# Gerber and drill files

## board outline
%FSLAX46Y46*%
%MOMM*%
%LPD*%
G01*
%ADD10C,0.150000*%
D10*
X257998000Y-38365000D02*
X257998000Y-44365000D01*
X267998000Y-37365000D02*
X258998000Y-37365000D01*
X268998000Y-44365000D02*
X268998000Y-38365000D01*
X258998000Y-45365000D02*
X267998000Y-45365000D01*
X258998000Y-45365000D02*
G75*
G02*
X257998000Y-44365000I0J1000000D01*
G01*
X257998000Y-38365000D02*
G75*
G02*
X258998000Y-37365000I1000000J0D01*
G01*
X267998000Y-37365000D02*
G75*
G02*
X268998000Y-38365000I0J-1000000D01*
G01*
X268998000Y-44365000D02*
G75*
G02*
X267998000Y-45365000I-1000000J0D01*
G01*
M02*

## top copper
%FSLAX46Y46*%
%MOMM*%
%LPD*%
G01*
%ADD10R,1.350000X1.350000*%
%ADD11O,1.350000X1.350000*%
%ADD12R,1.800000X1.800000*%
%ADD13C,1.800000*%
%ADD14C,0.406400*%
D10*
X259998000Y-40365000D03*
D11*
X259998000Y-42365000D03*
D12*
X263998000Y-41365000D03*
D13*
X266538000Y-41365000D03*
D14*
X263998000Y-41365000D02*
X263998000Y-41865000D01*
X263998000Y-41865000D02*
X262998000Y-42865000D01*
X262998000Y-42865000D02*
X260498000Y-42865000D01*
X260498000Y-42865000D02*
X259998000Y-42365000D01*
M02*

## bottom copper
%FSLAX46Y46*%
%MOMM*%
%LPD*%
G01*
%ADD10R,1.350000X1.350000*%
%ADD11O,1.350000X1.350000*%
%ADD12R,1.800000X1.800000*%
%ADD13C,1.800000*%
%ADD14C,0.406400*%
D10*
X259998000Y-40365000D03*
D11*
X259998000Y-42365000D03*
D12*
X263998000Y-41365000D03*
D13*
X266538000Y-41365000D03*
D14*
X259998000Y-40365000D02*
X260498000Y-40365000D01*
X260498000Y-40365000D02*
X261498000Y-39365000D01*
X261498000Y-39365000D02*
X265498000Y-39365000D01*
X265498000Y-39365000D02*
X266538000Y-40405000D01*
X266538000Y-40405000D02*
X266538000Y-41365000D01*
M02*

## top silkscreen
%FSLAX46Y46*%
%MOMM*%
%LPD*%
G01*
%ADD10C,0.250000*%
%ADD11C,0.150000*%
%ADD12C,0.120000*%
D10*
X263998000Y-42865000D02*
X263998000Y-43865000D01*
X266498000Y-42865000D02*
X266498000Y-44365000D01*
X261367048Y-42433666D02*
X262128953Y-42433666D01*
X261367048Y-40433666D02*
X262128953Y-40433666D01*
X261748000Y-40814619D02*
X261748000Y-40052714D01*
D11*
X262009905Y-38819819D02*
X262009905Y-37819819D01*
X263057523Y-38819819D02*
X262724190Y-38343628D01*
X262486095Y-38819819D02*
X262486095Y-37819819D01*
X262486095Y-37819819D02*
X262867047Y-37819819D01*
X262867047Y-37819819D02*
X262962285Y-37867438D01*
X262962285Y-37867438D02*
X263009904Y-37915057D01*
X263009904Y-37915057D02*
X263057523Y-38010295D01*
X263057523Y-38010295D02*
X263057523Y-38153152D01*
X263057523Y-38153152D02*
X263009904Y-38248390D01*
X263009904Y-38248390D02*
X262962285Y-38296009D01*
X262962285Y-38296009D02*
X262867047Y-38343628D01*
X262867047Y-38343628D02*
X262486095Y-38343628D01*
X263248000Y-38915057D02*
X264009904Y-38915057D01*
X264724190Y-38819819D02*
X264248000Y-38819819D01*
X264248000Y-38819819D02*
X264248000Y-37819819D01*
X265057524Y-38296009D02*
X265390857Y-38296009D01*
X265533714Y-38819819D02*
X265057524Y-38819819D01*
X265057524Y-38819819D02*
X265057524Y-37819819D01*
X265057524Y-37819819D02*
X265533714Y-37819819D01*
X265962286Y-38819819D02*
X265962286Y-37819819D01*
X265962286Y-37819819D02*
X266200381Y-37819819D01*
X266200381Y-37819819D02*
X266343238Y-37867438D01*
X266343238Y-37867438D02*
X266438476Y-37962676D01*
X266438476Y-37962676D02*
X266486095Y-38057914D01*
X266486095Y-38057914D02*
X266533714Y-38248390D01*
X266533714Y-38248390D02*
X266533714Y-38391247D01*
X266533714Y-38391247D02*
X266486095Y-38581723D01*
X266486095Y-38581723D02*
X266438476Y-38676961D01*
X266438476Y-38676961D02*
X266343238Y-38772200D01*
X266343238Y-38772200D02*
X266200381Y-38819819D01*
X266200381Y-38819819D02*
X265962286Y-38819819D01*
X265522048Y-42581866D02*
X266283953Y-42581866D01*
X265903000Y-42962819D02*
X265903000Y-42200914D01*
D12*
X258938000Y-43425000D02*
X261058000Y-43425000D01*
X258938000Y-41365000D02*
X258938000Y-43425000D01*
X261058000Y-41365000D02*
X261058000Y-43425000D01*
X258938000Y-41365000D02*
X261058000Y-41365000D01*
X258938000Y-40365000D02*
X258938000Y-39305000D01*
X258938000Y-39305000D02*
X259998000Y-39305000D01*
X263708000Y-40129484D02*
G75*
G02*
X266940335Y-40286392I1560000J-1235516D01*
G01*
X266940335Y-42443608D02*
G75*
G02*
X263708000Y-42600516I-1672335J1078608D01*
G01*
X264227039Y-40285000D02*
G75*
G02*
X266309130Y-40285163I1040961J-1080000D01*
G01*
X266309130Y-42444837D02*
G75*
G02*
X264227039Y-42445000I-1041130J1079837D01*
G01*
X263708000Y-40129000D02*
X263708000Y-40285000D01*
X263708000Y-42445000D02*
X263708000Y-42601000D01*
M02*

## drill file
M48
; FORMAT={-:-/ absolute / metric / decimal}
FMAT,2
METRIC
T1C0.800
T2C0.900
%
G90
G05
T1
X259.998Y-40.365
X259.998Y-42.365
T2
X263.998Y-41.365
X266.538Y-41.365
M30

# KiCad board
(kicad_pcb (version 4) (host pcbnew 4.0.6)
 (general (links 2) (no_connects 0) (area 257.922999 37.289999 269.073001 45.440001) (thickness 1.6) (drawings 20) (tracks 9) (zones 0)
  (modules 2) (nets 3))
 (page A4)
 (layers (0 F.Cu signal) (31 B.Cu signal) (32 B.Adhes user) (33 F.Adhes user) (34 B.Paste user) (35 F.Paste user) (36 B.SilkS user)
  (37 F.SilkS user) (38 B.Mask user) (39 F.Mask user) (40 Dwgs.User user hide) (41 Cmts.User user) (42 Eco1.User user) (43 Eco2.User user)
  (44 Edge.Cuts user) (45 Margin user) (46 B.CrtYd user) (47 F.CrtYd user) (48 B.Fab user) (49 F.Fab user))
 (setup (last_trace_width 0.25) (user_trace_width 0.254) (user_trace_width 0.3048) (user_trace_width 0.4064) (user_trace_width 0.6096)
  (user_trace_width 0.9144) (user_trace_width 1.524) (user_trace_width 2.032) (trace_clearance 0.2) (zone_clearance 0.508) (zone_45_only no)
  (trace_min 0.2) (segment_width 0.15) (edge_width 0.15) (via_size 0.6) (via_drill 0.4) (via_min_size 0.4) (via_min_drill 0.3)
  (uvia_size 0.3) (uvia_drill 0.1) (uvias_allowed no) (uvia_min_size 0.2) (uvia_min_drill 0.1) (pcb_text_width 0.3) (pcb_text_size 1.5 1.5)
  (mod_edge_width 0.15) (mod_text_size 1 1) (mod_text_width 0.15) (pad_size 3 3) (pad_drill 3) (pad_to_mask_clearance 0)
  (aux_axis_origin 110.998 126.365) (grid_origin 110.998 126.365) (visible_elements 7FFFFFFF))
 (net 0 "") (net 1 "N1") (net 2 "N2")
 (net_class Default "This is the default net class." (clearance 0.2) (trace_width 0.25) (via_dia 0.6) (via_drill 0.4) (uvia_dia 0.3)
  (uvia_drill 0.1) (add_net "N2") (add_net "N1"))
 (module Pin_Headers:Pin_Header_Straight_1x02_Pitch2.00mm (layer F.Cu) (at 259.998 40.365)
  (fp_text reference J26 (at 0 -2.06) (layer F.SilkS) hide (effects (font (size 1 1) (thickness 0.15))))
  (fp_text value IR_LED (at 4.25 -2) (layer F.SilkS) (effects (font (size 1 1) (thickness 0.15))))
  (fp_line (start -1.06 3.06) (end 1.06 3.06) (layer F.SilkS) (width 0.12))
  (fp_line (start -1.06 1) (end -1.06 3.06) (layer F.SilkS) (width 0.12))
  (fp_line (start 1.06 1) (end 1.06 3.06) (layer F.SilkS) (width 0.12))
  (fp_line (start -1.06 1) (end 1.06 1) (layer F.SilkS) (width 0.12))
  (fp_line (start -1.06 0) (end -1.06 -1.06) (layer F.SilkS) (width 0.12))
  (fp_line (start -1.06 -1.06) (end 0 -1.06) (layer F.SilkS) (width 0.12))
  (pad 1 thru_hole rect (at 0 0) (size 1.35 1.35) (drill 0.8) (layers *.Cu *.Mask) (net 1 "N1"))
  (pad 2 thru_hole oval (at 0 2) (size 1.35 1.35) (drill 0.8) (layers *.Cu *.Mask) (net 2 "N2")))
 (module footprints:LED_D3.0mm (layer F.Cu) (at 263.998 41.365)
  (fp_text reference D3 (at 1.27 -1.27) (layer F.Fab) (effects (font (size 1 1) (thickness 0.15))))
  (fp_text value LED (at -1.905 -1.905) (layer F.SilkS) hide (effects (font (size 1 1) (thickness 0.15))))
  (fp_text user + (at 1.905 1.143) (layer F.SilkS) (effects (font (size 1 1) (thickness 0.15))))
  (fp_arc (start 1.27 0) (end -0.29 -1.235516) (angle 108.8) (layer F.SilkS) (width 0.12))
  (fp_arc (start 1.27 0) (end -0.29 1.235516) (angle -108.8) (layer F.SilkS) (width 0.12))
  (fp_arc (start 1.27 0) (end 0.229039 -1.08) (angle 87.9) (layer F.SilkS) (width 0.12))
  (fp_arc (start 1.27 0) (end 0.229039 1.08) (angle -87.9) (layer F.SilkS) (width 0.12))
  (fp_line (start -0.29 -1.236) (end -0.29 -1.08) (layer F.SilkS) (width 0.12))
  (fp_line (start -0.29 1.08) (end -0.29 1.236) (layer F.SilkS) (width 0.12))
  (pad 1 thru_hole rect (at 0 0) (size 1.8 1.8) (drill 0.9) (layers *.Cu *.Mask) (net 2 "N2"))
  (pad 2 thru_hole circle (at 2.54 0) (size 1.8 1.8) (drill 0.9) (layers *.Cu *.Mask) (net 1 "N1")))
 (gr_line (start 257.998 38.365) (end 257.998 44.365) (angle 90) (layer Edge.Cuts) (width 0.15))
 (gr_line (start 267.998 37.365) (end 258.998 37.365) (angle 90) (layer Edge.Cuts) (width 0.15))
 (gr_line (start 268.998 44.365) (end 268.998 38.365) (angle 90) (layer Edge.Cuts) (width 0.15))
 (gr_line (start 258.998 45.365) (end 267.998 45.365) (angle 90) (layer Edge.Cuts) (width 0.15))
 (gr_arc (start 258.998 44.365) (end 258.998 45.365) (angle 90) (layer Edge.Cuts) (width 0.15))
 (gr_arc (start 258.998 38.365) (end 257.998 38.365) (angle 90) (layer Edge.Cuts) (width 0.15))
 (gr_arc (start 267.998 38.365) (end 267.998 37.365) (angle 90) (layer Edge.Cuts) (width 0.15))
 (gr_arc (start 267.998 44.365) (end 268.998 44.365) (angle 90) (layer Edge.Cuts) (width 0.15))
 (gr_line (start 263.998 42.865) (end 263.998 43.865) (angle 90) (layer F.SilkS) (width 0.25))
 (gr_line (start 266.498 42.865) (end 266.498 44.365) (angle 90) (layer F.SilkS) (width 0.25))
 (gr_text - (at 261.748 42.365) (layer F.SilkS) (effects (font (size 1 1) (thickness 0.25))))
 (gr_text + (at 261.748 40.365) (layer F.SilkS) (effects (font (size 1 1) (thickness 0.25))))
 (segment (start 263.998 41.365) (end 263.998 41.865) (width 0.4064) (layer F.Cu) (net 2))
 (segment (start 263.998 41.865) (end 262.998 42.865) (width 0.4064) (layer F.Cu) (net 2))
 (segment (start 262.998 42.865) (end 260.498 42.865) (width 0.4064) (layer F.Cu) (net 2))
 (segment (start 260.498 42.865) (end 259.998 42.365) (width 0.4064) (layer F.Cu) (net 2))
 (segment (start 259.998 40.365) (end 260.498 40.365) (width 0.4064) (layer B.Cu) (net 1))
 (segment (start 260.498 40.365) (end 261.498 39.365) (width 0.4064) (layer B.Cu) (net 1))
 (segment (start 261.498 39.365) (end 265.498 39.365) (width 0.4064) (layer B.Cu) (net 1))
 (segment (start 265.498 39.365) (end 266.538 40.405) (width 0.4064) (layer B.Cu) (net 1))
 (segment (start 266.538 40.405) (end 266.538 41.365) (width 0.4064) (layer B.Cu) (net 1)))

